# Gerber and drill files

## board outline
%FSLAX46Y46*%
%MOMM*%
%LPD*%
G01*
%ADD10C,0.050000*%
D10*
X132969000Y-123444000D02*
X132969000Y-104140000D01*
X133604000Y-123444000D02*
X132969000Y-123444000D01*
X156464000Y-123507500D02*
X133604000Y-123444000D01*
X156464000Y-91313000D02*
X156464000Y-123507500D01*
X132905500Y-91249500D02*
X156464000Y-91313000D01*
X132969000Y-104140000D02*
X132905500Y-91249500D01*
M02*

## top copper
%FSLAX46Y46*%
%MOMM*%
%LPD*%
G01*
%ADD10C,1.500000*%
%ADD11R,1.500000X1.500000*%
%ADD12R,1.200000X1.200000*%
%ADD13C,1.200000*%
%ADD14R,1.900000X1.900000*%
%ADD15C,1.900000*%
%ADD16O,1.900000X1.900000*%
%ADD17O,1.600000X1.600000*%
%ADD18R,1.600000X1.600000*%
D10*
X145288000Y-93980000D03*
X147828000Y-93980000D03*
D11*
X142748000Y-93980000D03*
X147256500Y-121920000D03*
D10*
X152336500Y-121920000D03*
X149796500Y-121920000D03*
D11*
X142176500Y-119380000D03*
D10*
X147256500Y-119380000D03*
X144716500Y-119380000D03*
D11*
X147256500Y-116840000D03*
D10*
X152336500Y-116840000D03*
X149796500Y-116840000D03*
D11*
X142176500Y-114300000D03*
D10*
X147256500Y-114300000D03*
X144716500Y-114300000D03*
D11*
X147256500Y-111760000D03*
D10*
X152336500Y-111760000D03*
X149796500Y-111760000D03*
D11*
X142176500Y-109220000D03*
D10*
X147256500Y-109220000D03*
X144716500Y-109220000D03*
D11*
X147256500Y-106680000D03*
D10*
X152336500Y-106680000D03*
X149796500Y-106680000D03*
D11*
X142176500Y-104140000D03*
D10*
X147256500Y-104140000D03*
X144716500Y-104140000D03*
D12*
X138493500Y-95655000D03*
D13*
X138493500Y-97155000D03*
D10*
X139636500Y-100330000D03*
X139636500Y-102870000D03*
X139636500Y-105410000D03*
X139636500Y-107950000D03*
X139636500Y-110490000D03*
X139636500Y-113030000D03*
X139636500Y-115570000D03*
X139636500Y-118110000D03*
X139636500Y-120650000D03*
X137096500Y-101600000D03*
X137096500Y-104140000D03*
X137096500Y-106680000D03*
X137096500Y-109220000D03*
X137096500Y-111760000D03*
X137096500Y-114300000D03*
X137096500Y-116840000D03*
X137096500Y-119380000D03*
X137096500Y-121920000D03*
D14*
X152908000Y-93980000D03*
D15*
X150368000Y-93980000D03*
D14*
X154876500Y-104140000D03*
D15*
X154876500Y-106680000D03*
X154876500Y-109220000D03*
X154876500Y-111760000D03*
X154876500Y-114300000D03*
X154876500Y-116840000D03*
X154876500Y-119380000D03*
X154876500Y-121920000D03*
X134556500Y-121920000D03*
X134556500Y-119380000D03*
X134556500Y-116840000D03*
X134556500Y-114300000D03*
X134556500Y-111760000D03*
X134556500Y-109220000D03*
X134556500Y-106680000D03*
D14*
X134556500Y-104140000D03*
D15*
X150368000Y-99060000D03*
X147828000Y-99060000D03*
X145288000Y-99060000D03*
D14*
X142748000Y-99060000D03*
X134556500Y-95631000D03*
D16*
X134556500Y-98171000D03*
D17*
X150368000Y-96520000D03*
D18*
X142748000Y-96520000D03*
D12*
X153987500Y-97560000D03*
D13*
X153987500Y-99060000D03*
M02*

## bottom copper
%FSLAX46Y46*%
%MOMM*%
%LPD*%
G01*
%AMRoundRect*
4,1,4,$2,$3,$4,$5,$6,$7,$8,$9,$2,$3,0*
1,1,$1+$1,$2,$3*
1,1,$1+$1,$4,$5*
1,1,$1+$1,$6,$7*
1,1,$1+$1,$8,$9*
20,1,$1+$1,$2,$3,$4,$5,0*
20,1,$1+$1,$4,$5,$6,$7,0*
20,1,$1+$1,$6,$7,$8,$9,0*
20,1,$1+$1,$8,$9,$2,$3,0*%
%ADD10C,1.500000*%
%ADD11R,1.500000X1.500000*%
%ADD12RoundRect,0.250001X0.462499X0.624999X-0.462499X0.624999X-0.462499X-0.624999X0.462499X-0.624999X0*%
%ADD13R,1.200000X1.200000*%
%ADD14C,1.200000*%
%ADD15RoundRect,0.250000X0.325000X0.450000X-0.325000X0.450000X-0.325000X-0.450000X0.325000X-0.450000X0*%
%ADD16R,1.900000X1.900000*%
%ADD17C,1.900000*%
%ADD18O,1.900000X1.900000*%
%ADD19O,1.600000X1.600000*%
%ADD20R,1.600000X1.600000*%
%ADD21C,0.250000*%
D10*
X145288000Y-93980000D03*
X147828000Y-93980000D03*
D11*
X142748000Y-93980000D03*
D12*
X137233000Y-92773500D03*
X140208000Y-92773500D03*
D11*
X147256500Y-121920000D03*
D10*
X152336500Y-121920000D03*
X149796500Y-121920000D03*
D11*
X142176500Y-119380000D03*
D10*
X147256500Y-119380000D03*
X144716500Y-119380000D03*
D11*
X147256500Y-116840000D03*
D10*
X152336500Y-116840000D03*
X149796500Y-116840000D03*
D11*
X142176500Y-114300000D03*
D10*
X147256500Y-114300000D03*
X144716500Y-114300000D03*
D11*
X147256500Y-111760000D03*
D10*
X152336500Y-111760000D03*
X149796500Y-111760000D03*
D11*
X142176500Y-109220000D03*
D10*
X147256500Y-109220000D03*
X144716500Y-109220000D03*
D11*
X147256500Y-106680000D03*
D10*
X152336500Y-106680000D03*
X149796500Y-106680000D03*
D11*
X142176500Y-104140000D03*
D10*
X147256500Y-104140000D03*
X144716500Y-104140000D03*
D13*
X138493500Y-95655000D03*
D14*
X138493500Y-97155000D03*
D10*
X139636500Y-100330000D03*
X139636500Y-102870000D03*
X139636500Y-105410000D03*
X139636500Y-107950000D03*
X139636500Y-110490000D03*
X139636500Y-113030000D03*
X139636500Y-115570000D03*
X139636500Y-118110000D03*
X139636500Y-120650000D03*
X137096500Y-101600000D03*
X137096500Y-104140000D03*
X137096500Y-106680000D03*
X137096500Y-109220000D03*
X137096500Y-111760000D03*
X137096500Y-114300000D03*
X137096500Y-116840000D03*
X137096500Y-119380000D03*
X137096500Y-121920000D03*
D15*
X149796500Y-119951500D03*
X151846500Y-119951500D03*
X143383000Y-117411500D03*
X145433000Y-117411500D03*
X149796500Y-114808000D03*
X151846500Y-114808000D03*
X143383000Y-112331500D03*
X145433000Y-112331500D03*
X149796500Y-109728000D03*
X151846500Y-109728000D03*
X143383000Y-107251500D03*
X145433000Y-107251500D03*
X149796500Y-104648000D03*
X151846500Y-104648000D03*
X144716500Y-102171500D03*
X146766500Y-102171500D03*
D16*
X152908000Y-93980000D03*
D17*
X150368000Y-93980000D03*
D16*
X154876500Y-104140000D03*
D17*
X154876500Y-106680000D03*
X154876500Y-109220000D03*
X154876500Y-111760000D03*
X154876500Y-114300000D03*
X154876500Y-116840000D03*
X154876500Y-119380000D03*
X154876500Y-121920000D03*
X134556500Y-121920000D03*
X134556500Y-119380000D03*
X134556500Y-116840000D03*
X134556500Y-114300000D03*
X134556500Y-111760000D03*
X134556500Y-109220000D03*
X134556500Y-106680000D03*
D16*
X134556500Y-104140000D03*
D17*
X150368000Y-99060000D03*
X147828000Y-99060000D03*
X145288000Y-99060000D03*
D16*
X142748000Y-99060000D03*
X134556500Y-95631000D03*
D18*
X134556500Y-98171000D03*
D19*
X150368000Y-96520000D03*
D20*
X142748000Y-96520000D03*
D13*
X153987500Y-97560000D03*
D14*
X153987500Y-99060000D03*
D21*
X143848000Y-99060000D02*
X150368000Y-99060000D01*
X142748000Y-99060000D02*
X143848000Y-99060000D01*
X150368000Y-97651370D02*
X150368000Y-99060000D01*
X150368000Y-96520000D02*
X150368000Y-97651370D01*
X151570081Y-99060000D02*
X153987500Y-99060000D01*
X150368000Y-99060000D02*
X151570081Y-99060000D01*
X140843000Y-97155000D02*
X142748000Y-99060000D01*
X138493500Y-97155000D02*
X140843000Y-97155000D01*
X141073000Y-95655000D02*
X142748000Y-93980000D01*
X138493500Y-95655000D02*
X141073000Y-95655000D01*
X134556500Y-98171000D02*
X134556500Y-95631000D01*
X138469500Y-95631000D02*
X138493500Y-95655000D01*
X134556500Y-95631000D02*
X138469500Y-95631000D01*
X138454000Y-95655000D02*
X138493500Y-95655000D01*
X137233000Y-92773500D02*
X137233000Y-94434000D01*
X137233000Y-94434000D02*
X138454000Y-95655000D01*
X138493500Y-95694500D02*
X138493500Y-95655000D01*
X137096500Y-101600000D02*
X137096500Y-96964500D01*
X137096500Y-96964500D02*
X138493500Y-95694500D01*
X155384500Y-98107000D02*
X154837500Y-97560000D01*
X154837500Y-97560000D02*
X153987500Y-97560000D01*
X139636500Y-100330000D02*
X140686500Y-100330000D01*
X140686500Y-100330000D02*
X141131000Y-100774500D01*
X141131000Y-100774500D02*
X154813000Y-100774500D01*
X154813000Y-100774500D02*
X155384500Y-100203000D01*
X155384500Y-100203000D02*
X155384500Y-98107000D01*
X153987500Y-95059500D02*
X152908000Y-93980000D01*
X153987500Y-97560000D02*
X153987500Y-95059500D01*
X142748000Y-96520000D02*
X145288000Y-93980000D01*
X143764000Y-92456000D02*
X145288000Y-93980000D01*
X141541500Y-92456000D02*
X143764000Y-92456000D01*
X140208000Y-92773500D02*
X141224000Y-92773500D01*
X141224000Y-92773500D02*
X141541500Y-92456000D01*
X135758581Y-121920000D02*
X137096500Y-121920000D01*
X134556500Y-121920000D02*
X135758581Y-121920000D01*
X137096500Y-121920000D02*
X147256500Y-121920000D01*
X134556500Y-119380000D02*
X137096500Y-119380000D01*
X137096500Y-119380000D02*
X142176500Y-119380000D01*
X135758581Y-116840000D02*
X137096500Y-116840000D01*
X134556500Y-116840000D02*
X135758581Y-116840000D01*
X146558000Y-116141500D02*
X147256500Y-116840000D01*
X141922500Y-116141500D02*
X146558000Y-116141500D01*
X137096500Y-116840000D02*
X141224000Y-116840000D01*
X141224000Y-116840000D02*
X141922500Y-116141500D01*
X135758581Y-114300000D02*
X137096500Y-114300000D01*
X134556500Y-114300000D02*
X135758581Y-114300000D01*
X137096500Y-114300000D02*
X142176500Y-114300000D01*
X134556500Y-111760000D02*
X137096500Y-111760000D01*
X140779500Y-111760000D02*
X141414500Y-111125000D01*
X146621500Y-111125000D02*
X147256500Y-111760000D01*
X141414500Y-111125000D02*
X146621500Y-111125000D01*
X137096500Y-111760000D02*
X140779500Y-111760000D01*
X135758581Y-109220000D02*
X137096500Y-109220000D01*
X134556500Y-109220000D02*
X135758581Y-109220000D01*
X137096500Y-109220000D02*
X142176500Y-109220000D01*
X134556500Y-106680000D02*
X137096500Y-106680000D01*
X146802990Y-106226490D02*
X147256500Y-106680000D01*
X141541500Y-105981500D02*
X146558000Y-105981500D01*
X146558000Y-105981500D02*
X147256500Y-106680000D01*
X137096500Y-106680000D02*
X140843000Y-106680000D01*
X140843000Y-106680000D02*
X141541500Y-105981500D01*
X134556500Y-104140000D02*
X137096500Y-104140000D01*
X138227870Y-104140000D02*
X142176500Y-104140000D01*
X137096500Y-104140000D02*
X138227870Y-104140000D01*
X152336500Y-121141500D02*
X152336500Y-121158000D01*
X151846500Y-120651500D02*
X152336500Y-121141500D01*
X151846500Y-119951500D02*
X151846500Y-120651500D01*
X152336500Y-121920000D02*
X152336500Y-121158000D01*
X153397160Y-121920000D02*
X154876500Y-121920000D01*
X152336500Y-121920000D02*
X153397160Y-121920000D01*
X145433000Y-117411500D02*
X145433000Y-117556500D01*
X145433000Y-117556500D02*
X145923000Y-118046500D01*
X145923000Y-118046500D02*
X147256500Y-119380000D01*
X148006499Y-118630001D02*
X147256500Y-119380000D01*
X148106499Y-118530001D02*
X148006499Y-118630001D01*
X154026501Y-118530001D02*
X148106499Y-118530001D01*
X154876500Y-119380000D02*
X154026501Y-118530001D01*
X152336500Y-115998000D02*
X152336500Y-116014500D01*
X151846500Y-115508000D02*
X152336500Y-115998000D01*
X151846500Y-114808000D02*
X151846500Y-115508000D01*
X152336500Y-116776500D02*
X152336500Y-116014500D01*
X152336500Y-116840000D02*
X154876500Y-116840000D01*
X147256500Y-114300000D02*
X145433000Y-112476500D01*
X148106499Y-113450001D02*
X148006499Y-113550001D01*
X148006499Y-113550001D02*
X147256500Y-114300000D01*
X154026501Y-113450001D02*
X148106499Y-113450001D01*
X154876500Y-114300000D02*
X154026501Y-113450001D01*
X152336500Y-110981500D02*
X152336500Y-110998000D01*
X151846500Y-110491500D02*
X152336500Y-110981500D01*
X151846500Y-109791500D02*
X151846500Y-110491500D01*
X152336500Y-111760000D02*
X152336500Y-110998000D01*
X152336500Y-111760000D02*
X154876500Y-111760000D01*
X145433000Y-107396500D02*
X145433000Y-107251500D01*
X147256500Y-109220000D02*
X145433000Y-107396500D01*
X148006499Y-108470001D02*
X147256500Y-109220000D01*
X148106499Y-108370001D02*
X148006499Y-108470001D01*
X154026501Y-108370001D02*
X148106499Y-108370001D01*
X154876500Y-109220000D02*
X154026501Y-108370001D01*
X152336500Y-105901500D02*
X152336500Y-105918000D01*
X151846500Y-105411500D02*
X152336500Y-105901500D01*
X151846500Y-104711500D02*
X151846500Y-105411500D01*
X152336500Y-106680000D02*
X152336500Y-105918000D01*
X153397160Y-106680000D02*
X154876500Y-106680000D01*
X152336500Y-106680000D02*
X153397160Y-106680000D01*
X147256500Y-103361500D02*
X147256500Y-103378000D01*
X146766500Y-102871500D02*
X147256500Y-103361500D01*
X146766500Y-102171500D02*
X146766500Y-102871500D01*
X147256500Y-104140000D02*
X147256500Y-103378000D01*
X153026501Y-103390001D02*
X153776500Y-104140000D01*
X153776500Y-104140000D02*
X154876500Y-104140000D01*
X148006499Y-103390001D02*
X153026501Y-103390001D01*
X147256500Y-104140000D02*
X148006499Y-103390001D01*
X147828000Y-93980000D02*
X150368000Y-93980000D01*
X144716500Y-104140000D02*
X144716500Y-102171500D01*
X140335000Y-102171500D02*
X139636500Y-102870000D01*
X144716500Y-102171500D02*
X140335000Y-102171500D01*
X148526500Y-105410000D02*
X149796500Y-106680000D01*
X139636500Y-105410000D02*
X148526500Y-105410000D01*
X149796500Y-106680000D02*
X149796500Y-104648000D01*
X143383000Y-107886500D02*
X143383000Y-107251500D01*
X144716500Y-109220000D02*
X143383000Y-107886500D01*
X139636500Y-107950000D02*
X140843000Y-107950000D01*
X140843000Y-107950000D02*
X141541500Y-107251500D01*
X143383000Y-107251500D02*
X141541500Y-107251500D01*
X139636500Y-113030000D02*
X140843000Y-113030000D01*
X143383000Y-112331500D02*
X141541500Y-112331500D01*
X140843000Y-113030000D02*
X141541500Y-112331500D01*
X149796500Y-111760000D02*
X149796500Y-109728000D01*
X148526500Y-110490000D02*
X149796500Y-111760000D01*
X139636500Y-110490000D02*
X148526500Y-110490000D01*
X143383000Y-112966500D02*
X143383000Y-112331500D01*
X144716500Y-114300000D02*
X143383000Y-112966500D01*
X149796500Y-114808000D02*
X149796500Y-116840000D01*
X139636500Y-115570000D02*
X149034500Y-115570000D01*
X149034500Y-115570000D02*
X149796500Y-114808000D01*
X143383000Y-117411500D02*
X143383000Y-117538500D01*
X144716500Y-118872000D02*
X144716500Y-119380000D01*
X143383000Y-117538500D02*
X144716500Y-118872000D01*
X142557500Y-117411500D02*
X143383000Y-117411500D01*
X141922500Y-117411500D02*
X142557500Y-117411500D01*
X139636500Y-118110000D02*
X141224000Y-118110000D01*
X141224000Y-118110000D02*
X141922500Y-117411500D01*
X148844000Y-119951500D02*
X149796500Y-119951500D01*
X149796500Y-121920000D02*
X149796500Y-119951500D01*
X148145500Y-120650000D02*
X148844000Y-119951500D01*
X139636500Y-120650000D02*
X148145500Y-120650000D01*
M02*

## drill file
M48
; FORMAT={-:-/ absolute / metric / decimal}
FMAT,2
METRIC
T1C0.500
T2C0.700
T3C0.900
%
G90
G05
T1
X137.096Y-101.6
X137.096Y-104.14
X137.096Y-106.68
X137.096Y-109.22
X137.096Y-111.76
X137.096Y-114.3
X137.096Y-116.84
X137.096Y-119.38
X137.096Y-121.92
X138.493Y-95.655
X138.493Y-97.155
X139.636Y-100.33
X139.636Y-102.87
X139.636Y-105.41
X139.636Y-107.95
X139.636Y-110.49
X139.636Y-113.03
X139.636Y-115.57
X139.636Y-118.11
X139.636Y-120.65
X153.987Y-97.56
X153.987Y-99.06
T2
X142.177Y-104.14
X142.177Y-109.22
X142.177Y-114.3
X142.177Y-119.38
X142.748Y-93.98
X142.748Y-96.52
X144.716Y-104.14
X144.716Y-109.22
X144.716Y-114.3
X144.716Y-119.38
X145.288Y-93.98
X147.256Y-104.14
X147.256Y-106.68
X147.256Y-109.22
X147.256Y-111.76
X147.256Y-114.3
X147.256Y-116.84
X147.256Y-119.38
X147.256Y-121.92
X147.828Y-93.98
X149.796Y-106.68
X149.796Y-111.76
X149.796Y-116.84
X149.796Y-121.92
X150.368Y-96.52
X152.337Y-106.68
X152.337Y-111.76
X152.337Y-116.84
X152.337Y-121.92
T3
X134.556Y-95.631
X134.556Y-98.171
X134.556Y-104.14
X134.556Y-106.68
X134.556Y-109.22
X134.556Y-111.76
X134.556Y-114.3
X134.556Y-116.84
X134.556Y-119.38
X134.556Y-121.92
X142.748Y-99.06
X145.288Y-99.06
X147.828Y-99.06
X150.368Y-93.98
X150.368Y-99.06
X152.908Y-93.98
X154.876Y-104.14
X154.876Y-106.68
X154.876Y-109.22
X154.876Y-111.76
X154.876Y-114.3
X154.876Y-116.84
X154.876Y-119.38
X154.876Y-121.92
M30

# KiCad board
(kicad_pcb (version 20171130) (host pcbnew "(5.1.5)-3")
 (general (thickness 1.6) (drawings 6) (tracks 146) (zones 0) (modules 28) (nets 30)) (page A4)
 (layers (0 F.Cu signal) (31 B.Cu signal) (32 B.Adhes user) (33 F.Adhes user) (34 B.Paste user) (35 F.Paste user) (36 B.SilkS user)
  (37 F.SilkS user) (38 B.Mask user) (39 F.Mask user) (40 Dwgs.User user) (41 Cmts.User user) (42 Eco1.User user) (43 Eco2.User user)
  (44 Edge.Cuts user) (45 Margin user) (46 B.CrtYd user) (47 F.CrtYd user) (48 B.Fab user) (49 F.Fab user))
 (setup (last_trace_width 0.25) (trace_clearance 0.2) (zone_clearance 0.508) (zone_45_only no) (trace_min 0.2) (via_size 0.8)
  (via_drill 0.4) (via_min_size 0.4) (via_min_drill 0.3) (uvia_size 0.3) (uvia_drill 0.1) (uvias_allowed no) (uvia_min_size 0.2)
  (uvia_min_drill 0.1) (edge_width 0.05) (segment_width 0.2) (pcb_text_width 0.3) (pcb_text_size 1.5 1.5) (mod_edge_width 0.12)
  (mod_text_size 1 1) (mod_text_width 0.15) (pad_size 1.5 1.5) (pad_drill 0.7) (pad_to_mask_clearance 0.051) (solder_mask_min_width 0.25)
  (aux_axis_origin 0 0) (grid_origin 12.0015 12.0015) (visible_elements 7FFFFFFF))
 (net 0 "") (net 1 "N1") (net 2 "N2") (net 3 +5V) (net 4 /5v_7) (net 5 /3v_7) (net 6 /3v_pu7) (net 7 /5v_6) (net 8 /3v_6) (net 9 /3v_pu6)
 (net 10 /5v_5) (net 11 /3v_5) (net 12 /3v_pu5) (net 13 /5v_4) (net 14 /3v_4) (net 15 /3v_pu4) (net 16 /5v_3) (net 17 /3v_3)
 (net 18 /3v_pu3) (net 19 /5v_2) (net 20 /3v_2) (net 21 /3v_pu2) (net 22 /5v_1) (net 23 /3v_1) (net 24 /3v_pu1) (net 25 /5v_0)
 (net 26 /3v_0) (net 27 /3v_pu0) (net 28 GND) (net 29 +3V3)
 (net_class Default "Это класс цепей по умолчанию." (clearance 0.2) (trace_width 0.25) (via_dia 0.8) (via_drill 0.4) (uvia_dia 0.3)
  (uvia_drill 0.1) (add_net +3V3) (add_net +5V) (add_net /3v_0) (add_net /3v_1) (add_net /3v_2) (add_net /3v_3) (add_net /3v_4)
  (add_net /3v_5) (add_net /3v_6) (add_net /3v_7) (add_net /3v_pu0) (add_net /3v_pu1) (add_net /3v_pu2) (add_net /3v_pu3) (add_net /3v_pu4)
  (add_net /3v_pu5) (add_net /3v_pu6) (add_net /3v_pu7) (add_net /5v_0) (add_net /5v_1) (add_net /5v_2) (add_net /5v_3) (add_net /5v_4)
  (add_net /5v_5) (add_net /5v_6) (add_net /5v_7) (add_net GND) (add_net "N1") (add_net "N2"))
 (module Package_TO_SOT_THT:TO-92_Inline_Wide (layer F.Cu) (at 142.748 93.98)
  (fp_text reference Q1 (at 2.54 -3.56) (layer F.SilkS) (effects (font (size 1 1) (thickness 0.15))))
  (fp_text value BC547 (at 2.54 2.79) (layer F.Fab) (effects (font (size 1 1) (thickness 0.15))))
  (pad 2 thru_hole circle (at 2.54 0 90) (size 1.5 1.5) (drill 0.7) (layers *.Cu *.Mask) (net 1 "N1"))
  (pad 3 thru_hole circle (at 5.08 0 90) (size 1.5 1.5) (drill 0.7) (layers *.Cu *.Mask) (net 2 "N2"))
  (pad 1 thru_hole rect (at 0 0 90) (size 1.5 1.5) (drill 0.7) (layers *.Cu *.Mask) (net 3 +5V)))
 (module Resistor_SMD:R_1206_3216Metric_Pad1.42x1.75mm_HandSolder (layer B.Cu) (at 138.7205 92.7735 180)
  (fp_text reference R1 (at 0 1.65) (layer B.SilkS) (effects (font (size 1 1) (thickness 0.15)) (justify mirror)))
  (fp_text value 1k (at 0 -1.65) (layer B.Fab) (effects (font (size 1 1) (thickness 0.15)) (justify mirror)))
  (pad 2 smd roundrect (at 1.4875 0 180) (size 1.425 1.75) (layers B.Cu B.Paste B.Mask) (roundrect_rratio 0.175439) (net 3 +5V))
  (pad 1 smd roundrect (at -1.4875 0 180) (size 1.425 1.75) (layers B.Cu B.Paste B.Mask) (roundrect_rratio 0.175439) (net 1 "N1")))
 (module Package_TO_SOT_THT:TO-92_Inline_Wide (layer F.Cu) (at 147.2565 121.92)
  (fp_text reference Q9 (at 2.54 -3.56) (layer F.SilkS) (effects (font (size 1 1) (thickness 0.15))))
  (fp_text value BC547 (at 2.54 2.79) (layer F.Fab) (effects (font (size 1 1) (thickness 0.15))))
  (pad 1 thru_hole rect (at 0 0 90) (size 1.5 1.5) (drill 0.7) (layers *.Cu *.Mask) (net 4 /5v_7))
  (pad 3 thru_hole circle (at 5.08 0 90) (size 1.5 1.5) (drill 0.7) (layers *.Cu *.Mask) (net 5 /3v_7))
  (pad 2 thru_hole circle (at 2.54 0 90) (size 1.5 1.5) (drill 0.7) (layers *.Cu *.Mask) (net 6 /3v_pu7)))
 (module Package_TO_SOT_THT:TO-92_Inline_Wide (layer F.Cu) (at 142.1765 119.38)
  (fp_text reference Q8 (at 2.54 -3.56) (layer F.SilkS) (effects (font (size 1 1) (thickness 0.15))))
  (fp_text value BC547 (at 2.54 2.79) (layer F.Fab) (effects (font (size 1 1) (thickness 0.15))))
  (pad 1 thru_hole rect (at 0 0 90) (size 1.5 1.5) (drill 0.7) (layers *.Cu *.Mask) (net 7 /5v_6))
  (pad 3 thru_hole circle (at 5.08 0 90) (size 1.5 1.5) (drill 0.7) (layers *.Cu *.Mask) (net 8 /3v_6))
  (pad 2 thru_hole circle (at 2.54 0 90) (size 1.5 1.5) (drill 0.7) (layers *.Cu *.Mask) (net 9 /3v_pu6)))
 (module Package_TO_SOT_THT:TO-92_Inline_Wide (layer F.Cu) (at 147.2565 116.84)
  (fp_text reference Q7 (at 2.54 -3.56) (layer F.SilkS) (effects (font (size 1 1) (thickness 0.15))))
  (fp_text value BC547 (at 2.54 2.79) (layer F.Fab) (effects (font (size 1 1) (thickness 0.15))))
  (pad 1 thru_hole rect (at 0 0 90) (size 1.5 1.5) (drill 0.7) (layers *.Cu *.Mask) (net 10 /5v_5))
  (pad 3 thru_hole circle (at 5.08 0 90) (size 1.5 1.5) (drill 0.7) (layers *.Cu *.Mask) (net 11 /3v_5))
  (pad 2 thru_hole circle (at 2.54 0 90) (size 1.5 1.5) (drill 0.7) (layers *.Cu *.Mask) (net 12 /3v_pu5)))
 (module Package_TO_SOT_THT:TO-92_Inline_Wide (layer F.Cu) (at 142.1765 114.3)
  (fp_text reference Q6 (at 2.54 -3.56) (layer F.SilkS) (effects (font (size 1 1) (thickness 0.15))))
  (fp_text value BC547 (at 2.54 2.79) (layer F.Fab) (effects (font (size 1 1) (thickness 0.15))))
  (pad 1 thru_hole rect (at 0 0 90) (size 1.5 1.5) (drill 0.7) (layers *.Cu *.Mask) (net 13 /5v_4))
  (pad 3 thru_hole circle (at 5.08 0 90) (size 1.5 1.5) (drill 0.7) (layers *.Cu *.Mask) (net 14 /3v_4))
  (pad 2 thru_hole circle (at 2.54 0 90) (size 1.5 1.5) (drill 0.7) (layers *.Cu *.Mask) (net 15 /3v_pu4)))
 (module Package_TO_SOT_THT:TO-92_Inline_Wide (layer F.Cu) (at 147.2565 111.76)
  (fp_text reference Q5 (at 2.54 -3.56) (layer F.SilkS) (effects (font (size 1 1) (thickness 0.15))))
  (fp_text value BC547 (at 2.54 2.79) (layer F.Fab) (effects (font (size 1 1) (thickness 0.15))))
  (pad 1 thru_hole rect (at 0 0 90) (size 1.5 1.5) (drill 0.7) (layers *.Cu *.Mask) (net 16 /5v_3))
  (pad 3 thru_hole circle (at 5.08 0 90) (size 1.5 1.5) (drill 0.7) (layers *.Cu *.Mask) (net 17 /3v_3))
  (pad 2 thru_hole circle (at 2.54 0 90) (size 1.5 1.5) (drill 0.7) (layers *.Cu *.Mask) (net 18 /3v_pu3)))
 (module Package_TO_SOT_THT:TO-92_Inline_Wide (layer F.Cu) (at 142.1765 109.22)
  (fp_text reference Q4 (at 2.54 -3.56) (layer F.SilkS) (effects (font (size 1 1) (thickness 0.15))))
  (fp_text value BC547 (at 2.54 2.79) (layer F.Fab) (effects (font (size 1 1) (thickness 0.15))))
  (pad 1 thru_hole rect (at 0 0 90) (size 1.5 1.5) (drill 0.7) (layers *.Cu *.Mask) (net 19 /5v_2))
  (pad 3 thru_hole circle (at 5.08 0 90) (size 1.5 1.5) (drill 0.7) (layers *.Cu *.Mask) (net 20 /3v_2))
  (pad 2 thru_hole circle (at 2.54 0 90) (size 1.5 1.5) (drill 0.7) (layers *.Cu *.Mask) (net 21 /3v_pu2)))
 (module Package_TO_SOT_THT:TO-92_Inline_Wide (layer F.Cu) (at 147.2565 106.68)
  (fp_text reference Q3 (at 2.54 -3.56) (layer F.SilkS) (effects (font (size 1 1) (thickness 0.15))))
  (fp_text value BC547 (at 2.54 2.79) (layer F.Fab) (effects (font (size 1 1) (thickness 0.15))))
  (pad 1 thru_hole rect (at 0 0 90) (size 1.5 1.5) (drill 0.7) (layers *.Cu *.Mask) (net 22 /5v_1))
  (pad 3 thru_hole circle (at 5.08 0 90) (size 1.5 1.5) (drill 0.7) (layers *.Cu *.Mask) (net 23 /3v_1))
  (pad 2 thru_hole circle (at 2.54 0 90) (size 1.5 1.5) (drill 0.7) (layers *.Cu *.Mask) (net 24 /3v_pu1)))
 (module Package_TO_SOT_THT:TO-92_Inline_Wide (layer F.Cu) (at 142.1765 104.14)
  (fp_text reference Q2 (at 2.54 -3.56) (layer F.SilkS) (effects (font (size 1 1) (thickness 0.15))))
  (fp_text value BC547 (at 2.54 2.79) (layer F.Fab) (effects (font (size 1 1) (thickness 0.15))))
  (pad 1 thru_hole rect (at 0 0 90) (size 1.5 1.5) (drill 0.7) (layers *.Cu *.Mask) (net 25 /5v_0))
  (pad 3 thru_hole circle (at 5.08 0 90) (size 1.5 1.5) (drill 0.7) (layers *.Cu *.Mask) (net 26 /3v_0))
  (pad 2 thru_hole circle (at 2.54 0 90) (size 1.5 1.5) (drill 0.7) (layers *.Cu *.Mask) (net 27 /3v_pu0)))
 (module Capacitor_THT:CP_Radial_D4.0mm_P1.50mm (layer F.Cu) (at 138.4935 95.655 270)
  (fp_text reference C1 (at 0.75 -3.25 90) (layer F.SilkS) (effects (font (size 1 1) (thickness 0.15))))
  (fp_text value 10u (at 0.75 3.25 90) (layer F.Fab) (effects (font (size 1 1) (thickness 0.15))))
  (pad 1 thru_hole rect (at 0 0 270) (size 1.2 1.2) (drill 0.5) (layers *.Cu *.Mask) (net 3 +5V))
  (pad 2 thru_hole circle (at 1.5 0 270) (size 1.2 1.2) (drill 0.5) (layers *.Cu *.Mask) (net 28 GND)))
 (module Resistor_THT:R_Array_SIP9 (layer F.Cu) (at 139.6365 100.33 270)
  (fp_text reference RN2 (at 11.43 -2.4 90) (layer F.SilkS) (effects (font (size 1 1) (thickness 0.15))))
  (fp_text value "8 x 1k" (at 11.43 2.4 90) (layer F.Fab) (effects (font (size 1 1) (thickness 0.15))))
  (pad 1 thru_hole circle (at 0 0 270) (size 1.5 1.5) (drill 0.5) (layers *.Cu *.Mask) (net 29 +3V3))
  (pad 2 thru_hole circle (at 2.54 0 270) (size 1.5 1.5) (drill 0.5) (layers *.Cu *.Mask) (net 27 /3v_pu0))
  (pad 3 thru_hole circle (at 5.08 0 270) (size 1.5 1.5) (drill 0.5) (layers *.Cu *.Mask) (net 24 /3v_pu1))
  (pad 4 thru_hole circle (at 7.62 0 270) (size 1.5 1.5) (drill 0.5) (layers *.Cu *.Mask) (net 21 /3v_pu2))
  (pad 5 thru_hole circle (at 10.16 0 270) (size 1.5 1.5) (drill 0.5) (layers *.Cu *.Mask) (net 18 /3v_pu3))
  (pad 6 thru_hole circle (at 12.7 0 270) (size 1.5 1.5) (drill 0.5) (layers *.Cu *.Mask) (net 15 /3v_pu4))
  (pad 7 thru_hole circle (at 15.24 0 270) (size 1.5 1.5) (drill 0.5) (layers *.Cu *.Mask) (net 12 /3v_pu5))
  (pad 8 thru_hole circle (at 17.78 0 270) (size 1.5 1.5) (drill 0.5) (layers *.Cu *.Mask) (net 9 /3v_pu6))
  (pad 9 thru_hole circle (at 20.32 0 270) (size 1.5 1.5) (drill 0.5) (layers *.Cu *.Mask) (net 6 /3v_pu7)))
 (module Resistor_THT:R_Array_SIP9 (layer F.Cu) (at 137.0965 101.6 270)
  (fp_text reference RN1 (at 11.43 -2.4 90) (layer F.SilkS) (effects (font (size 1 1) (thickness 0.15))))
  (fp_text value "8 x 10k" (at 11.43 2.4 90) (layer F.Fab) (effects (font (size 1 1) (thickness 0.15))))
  (pad 1 thru_hole circle (at 0 0 270) (size 1.5 1.5) (drill 0.5) (layers *.Cu *.Mask) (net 3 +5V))
  (pad 2 thru_hole circle (at 2.54 0 270) (size 1.5 1.5) (drill 0.5) (layers *.Cu *.Mask) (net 25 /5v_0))
  (pad 3 thru_hole circle (at 5.08 0 270) (size 1.5 1.5) (drill 0.5) (layers *.Cu *.Mask) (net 22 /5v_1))
  (pad 4 thru_hole circle (at 7.62 0 270) (size 1.5 1.5) (drill 0.5) (layers *.Cu *.Mask) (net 19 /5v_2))
  (pad 5 thru_hole circle (at 10.16 0 270) (size 1.5 1.5) (drill 0.5) (layers *.Cu *.Mask) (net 16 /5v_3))
  (pad 6 thru_hole circle (at 12.7 0 270) (size 1.5 1.5) (drill 0.5) (layers *.Cu *.Mask) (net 13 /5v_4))
  (pad 7 thru_hole circle (at 15.24 0 270) (size 1.5 1.5) (drill 0.5) (layers *.Cu *.Mask) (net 10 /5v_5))
  (pad 8 thru_hole circle (at 17.78 0 270) (size 1.5 1.5) (drill 0.5) (layers *.Cu *.Mask) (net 7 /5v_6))
  (pad 9 thru_hole circle (at 20.32 0 270) (size 1.5 1.5) (drill 0.5) (layers *.Cu *.Mask) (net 4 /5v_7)))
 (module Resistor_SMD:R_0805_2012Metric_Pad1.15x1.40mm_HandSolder (layer B.Cu) (at 150.8215 119.9515 180)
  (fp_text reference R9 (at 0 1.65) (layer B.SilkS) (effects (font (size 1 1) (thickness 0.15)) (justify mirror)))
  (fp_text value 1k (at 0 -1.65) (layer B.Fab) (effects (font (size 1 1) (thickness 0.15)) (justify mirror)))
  (pad 2 smd roundrect (at 1.025 0 180) (size 1.15 1.4) (layers B.Cu B.Paste B.Mask) (roundrect_rratio 0.217391) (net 6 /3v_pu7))
  (pad 1 smd roundrect (at -1.025 0 180) (size 1.15 1.4) (layers B.Cu B.Paste B.Mask) (roundrect_rratio 0.217391) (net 5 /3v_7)))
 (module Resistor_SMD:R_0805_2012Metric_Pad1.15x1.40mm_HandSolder (layer B.Cu) (at 144.408 117.4115 180)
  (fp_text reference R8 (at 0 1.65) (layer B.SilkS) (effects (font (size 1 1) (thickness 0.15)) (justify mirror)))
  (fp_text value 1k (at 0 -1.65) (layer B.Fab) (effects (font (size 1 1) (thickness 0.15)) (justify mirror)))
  (pad 2 smd roundrect (at 1.025 0 180) (size 1.15 1.4) (layers B.Cu B.Paste B.Mask) (roundrect_rratio 0.217391) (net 9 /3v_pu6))
  (pad 1 smd roundrect (at -1.025 0 180) (size 1.15 1.4) (layers B.Cu B.Paste B.Mask) (roundrect_rratio 0.217391) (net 8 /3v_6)))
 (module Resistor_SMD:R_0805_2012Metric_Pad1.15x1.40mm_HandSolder (layer B.Cu) (at 150.8215 114.808 180)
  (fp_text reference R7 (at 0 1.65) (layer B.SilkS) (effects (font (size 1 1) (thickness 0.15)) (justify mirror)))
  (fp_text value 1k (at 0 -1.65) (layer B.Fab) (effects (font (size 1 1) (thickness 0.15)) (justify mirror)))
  (pad 2 smd roundrect (at 1.025 0 180) (size 1.15 1.4) (layers B.Cu B.Paste B.Mask) (roundrect_rratio 0.217391) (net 12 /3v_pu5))
  (pad 1 smd roundrect (at -1.025 0 180) (size 1.15 1.4) (layers B.Cu B.Paste B.Mask) (roundrect_rratio 0.217391) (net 11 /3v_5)))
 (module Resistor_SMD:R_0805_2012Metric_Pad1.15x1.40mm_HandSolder (layer B.Cu) (at 144.408 112.3315 180)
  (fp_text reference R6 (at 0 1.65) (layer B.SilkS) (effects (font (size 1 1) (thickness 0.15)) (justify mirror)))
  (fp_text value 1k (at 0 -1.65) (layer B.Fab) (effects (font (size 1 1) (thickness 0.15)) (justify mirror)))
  (pad 2 smd roundrect (at 1.025 0 180) (size 1.15 1.4) (layers B.Cu B.Paste B.Mask) (roundrect_rratio 0.217391) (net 15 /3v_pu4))
  (pad 1 smd roundrect (at -1.025 0 180) (size 1.15 1.4) (layers B.Cu B.Paste B.Mask) (roundrect_rratio 0.217391) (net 14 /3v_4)))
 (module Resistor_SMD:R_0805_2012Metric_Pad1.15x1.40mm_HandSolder (layer B.Cu) (at 150.8215 109.728 180)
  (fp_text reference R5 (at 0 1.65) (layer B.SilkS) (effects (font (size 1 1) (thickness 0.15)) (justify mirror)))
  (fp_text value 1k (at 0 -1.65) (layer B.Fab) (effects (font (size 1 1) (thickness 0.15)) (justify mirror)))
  (pad 2 smd roundrect (at 1.025 0 180) (size 1.15 1.4) (layers B.Cu B.Paste B.Mask) (roundrect_rratio 0.217391) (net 18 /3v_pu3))
  (pad 1 smd roundrect (at -1.025 0 180) (size 1.15 1.4) (layers B.Cu B.Paste B.Mask) (roundrect_rratio 0.217391) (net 17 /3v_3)))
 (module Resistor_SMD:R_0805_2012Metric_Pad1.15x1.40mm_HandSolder (layer B.Cu) (at 144.408 107.2515 180)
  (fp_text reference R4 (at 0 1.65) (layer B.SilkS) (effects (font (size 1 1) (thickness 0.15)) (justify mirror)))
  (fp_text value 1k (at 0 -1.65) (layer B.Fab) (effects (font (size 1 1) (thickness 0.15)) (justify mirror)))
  (pad 2 smd roundrect (at 1.025 0 180) (size 1.15 1.4) (layers B.Cu B.Paste B.Mask) (roundrect_rratio 0.217391) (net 21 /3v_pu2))
  (pad 1 smd roundrect (at -1.025 0 180) (size 1.15 1.4) (layers B.Cu B.Paste B.Mask) (roundrect_rratio 0.217391) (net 20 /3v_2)))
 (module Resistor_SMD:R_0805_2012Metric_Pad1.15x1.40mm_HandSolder (layer B.Cu) (at 150.8215 104.648 180)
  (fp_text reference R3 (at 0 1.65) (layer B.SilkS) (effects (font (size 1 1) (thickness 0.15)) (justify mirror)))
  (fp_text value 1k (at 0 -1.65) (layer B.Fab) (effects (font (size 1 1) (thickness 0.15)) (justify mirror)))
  (pad 2 smd roundrect (at 1.025 0 180) (size 1.15 1.4) (layers B.Cu B.Paste B.Mask) (roundrect_rratio 0.217391) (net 24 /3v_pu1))
  (pad 1 smd roundrect (at -1.025 0 180) (size 1.15 1.4) (layers B.Cu B.Paste B.Mask) (roundrect_rratio 0.217391) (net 23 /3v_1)))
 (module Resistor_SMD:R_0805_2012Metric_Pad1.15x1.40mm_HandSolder (layer B.Cu) (at 145.7415 102.1715 180)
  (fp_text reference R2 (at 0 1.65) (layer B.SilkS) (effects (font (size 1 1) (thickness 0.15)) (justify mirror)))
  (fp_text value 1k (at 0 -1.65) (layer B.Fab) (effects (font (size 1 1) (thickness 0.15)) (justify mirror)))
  (pad 2 smd roundrect (at 1.025 0 180) (size 1.15 1.4) (layers B.Cu B.Paste B.Mask) (roundrect_rratio 0.217391) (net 27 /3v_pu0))
  (pad 1 smd roundrect (at -1.025 0 180) (size 1.15 1.4) (layers B.Cu B.Paste B.Mask) (roundrect_rratio 0.217391) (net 26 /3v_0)))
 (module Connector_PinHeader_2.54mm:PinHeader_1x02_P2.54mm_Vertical (layer F.Cu) (at 152.908 93.98 270)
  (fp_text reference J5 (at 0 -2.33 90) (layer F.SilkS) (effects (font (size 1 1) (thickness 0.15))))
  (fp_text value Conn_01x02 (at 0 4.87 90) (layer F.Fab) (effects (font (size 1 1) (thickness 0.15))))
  (pad 1 thru_hole rect (at 0 0 270) (size 1.9 1.9) (drill 0.9) (layers *.Cu *.Mask) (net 29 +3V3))
  (pad 2 thru_hole circle (at 0 2.54 270) (size 1.9 1.9) (drill 0.9) (layers *.Cu *.Mask) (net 2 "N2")))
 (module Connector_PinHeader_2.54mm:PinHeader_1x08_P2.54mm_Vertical (layer F.Cu) (at 154.8765 104.14)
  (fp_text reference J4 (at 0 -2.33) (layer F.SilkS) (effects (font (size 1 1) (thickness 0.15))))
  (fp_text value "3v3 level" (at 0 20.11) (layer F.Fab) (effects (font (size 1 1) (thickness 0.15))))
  (pad 1 thru_hole rect (at 0 0) (size 1.9 1.9) (drill 0.9) (layers *.Cu *.Mask) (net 26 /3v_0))
  (pad 2 thru_hole circle (at 0 2.54) (size 1.9 1.9) (drill 0.9) (layers *.Cu *.Mask) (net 23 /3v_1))
  (pad 3 thru_hole circle (at 0 5.08) (size 1.9 1.9) (drill 0.9) (layers *.Cu *.Mask) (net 20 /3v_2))
  (pad 4 thru_hole circle (at 0 7.62) (size 1.9 1.9) (drill 0.9) (layers *.Cu *.Mask) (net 17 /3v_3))
  (pad 5 thru_hole circle (at 0 10.16) (size 1.9 1.9) (drill 0.9) (layers *.Cu *.Mask) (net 14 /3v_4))
  (pad 6 thru_hole circle (at 0 12.7) (size 1.9 1.9) (drill 0.9) (layers *.Cu *.Mask) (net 11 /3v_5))
  (pad 7 thru_hole circle (at 0 15.24) (size 1.9 1.9) (drill 0.9) (layers *.Cu *.Mask) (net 8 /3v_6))
  (pad 8 thru_hole circle (at 0 17.78) (size 1.9 1.9) (drill 0.9) (layers *.Cu *.Mask) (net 5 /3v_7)))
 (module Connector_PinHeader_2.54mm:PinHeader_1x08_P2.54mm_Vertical (layer F.Cu) (at 134.5565 104.14)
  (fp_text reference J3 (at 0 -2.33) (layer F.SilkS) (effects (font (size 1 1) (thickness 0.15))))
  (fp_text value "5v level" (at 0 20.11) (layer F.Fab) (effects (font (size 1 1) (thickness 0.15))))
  (pad 8 thru_hole circle (at 0 17.78) (size 1.9 1.9) (drill 0.9) (layers *.Cu *.Mask) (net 4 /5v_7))
  (pad 7 thru_hole circle (at 0 15.24) (size 1.9 1.9) (drill 0.9) (layers *.Cu *.Mask) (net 7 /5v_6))
  (pad 6 thru_hole circle (at 0 12.7) (size 1.9 1.9) (drill 0.9) (layers *.Cu *.Mask) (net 10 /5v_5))
  (pad 5 thru_hole circle (at 0 10.16) (size 1.9 1.9) (drill 0.9) (layers *.Cu *.Mask) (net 13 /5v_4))
  (pad 4 thru_hole circle (at 0 7.62) (size 1.9 1.9) (drill 0.9) (layers *.Cu *.Mask) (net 16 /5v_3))
  (pad 3 thru_hole circle (at 0 5.08) (size 1.9 1.9) (drill 0.9) (layers *.Cu *.Mask) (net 19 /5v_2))
  (pad 2 thru_hole circle (at 0 2.54) (size 1.9 1.9) (drill 0.9) (layers *.Cu *.Mask) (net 22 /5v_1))
  (pad 1 thru_hole rect (at 0 0) (size 1.9 1.9) (drill 0.9) (layers *.Cu *.Mask) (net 25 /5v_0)))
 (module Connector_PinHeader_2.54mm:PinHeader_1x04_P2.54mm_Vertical (layer F.Cu) (at 142.748 99.06 90)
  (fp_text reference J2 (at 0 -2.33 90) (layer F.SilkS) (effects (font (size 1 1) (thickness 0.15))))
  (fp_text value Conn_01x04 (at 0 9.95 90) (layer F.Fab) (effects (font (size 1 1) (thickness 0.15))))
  (pad 4 thru_hole circle (at 0 7.62 90) (size 1.9 1.9) (drill 0.9) (layers *.Cu *.Mask) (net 28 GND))
  (pad 3 thru_hole circle (at 0 5.08 90) (size 1.9 1.9) (drill 0.9) (layers *.Cu *.Mask) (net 28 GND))
  (pad 2 thru_hole circle (at 0 2.54 90) (size 1.9 1.9) (drill 0.9) (layers *.Cu *.Mask) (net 28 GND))
  (pad 1 thru_hole rect (at 0 0 90) (size 1.9 1.9) (drill 0.9) (layers *.Cu *.Mask) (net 28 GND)))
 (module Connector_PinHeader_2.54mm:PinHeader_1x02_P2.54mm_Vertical (layer F.Cu) (at 134.5565 95.631)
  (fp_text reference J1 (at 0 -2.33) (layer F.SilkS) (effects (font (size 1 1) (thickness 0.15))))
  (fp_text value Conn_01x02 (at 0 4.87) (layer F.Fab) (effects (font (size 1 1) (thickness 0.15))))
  (pad 1 thru_hole rect (at 0 0) (size 1.9 1.9) (drill 0.9) (layers *.Cu *.Mask) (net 3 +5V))
  (pad 2 thru_hole oval (at 0 2.54) (size 1.9 1.9) (drill 0.9) (layers *.Cu *.Mask) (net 3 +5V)))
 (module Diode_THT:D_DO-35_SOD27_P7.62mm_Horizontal (layer F.Cu) (at 142.748 96.52)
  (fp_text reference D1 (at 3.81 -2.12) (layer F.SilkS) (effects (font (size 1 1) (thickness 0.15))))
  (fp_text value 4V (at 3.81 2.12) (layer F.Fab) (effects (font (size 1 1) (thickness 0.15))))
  (pad 2 thru_hole oval (at 7.62 0) (size 1.6 1.6) (drill 0.7) (layers *.Cu *.Mask) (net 28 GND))
  (pad 1 thru_hole rect (at 0 0) (size 1.6 1.6) (drill 0.7) (layers *.Cu *.Mask) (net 1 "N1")))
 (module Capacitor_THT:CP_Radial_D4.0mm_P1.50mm (layer F.Cu) (at 153.9875 97.56 270)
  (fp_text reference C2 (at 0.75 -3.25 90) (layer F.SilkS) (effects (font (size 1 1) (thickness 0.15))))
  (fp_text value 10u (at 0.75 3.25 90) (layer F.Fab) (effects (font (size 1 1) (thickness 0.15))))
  (pad 1 thru_hole rect (at 0 0 270) (size 1.2 1.2) (drill 0.5) (layers *.Cu *.Mask) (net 29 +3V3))
  (pad 2 thru_hole circle (at 1.5 0 270) (size 1.2 1.2) (drill 0.5) (layers *.Cu *.Mask) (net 28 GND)))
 (gr_line (start 132.969 123.444) (end 132.969 104.14) (layer Edge.Cuts) (width 0.05))
 (gr_line (start 133.604 123.444) (end 132.969 123.444) (layer Edge.Cuts) (width 0.05))
 (gr_line (start 156.464 123.5075) (end 133.604 123.444) (layer Edge.Cuts) (width 0.05))
 (gr_line (start 156.464 91.313) (end 156.464 123.5075) (layer Edge.Cuts) (width 0.05))
 (gr_line (start 132.9055 91.2495) (end 156.464 91.313) (layer Edge.Cuts) (width 0.05))
 (gr_line (start 132.969 104.14) (end 132.9055 91.2495) (layer Edge.Cuts) (width 0.05))
 (segment (start 143.848 99.06) (end 150.368 99.06) (width 0.25) (layer B.Cu) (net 28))
 (segment (start 142.748 99.06) (end 143.848 99.06) (width 0.25) (layer B.Cu) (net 28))
 (segment (start 150.368 97.65137) (end 150.368 99.06) (width 0.25) (layer B.Cu) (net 28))
 (segment (start 150.368 96.52) (end 150.368 97.65137) (width 0.25) (layer B.Cu) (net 28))
 (segment (start 151.570081 99.06) (end 153.9875 99.06) (width 0.25) (layer B.Cu) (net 28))
 (segment (start 150.368 99.06) (end 151.570081 99.06) (width 0.25) (layer B.Cu) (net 28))
 (segment (start 140.843 97.155) (end 142.748 99.06) (width 0.25) (layer B.Cu) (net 28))
 (segment (start 138.4935 97.155) (end 140.843 97.155) (width 0.25) (layer B.Cu) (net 28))
 (segment (start 141.073 95.655) (end 142.748 93.98) (width 0.25) (layer B.Cu) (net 3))
 (segment (start 138.4935 95.655) (end 141.073 95.655) (width 0.25) (layer B.Cu) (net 3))
 (segment (start 134.5565 98.171) (end 134.5565 95.631) (width 0.25) (layer B.Cu) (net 3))
 (segment (start 138.4695 95.631) (end 138.4935 95.655) (width 0.25) (layer B.Cu) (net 3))
 (segment (start 134.5565 95.631) (end 138.4695 95.631) (width 0.25) (layer B.Cu) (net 3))
 (segment (start 138.454 95.655) (end 138.4935 95.655) (width 0.25) (layer B.Cu) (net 3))
 (segment (start 137.233 92.7735) (end 137.233 94.434) (width 0.25) (layer B.Cu) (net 3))
 (segment (start 137.233 94.434) (end 138.454 95.655) (width 0.25) (layer B.Cu) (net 3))
 (segment (start 138.4935 95.6945) (end 138.4935 95.655) (width 0.25) (layer B.Cu) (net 3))
 (segment (start 137.0965 101.6) (end 137.0965 96.9645) (width 0.25) (layer B.Cu) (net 3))
 (segment (start 137.0965 96.9645) (end 138.4935 95.6945) (width 0.25) (layer B.Cu) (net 3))
 (segment (start 155.3845 98.107) (end 154.8375 97.56) (width 0.25) (layer B.Cu) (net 29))
 (segment (start 154.8375 97.56) (end 153.9875 97.56) (width 0.25) (layer B.Cu) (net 29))
 (segment (start 139.6365 100.33) (end 140.6865 100.33) (width 0.25) (layer B.Cu) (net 29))
 (segment (start 140.6865 100.33) (end 141.131 100.7745) (width 0.25) (layer B.Cu) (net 29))
 (segment (start 141.131 100.7745) (end 154.813 100.7745) (width 0.25) (layer B.Cu) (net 29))
 (segment (start 154.813 100.7745) (end 155.3845 100.203) (width 0.25) (layer B.Cu) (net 29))
 (segment (start 155.3845 100.203) (end 155.3845 98.107) (width 0.25) (layer B.Cu) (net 29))
 (segment (start 153.9875 95.0595) (end 152.908 93.98) (width 0.25) (layer B.Cu) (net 29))
 (segment (start 153.9875 97.56) (end 153.9875 95.0595) (width 0.25) (layer B.Cu) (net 29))
 (segment (start 142.748 96.52) (end 145.288 93.98) (width 0.25) (layer B.Cu) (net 1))
 (segment (start 143.764 92.456) (end 145.288 93.98) (width 0.25) (layer B.Cu) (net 1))
 (segment (start 141.5415 92.456) (end 143.764 92.456) (width 0.25) (layer B.Cu) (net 1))
 (segment (start 140.208 92.7735) (end 141.224 92.7735) (width 0.25) (layer B.Cu) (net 1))
 (segment (start 141.224 92.7735) (end 141.5415 92.456) (width 0.25) (layer B.Cu) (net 1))
 (segment (start 135.758581 121.92) (end 137.0965 121.92) (width 0.25) (layer B.Cu) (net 4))
 (segment (start 134.5565 121.92) (end 135.758581 121.92) (width 0.25) (layer B.Cu) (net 4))
 (segment (start 137.0965 121.92) (end 147.2565 121.92) (width 0.25) (layer B.Cu) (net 4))
 (segment (start 134.5565 119.38) (end 137.0965 119.38) (width 0.25) (layer B.Cu) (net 7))
 (segment (start 137.0965 119.38) (end 142.1765 119.38) (width 0.25) (layer B.Cu) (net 7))
 (segment (start 135.758581 116.84) (end 137.0965 116.84) (width 0.25) (layer B.Cu) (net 10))
 (segment (start 134.5565 116.84) (end 135.758581 116.84) (width 0.25) (layer B.Cu) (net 10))
 (segment (start 146.558 116.1415) (end 147.2565 116.84) (width 0.25) (layer B.Cu) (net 10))
 (segment (start 141.9225 116.1415) (end 146.558 116.1415) (width 0.25) (layer B.Cu) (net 10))
 (segment (start 137.0965 116.84) (end 141.224 116.84) (width 0.25) (layer B.Cu) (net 10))
 (segment (start 141.224 116.84) (end 141.9225 116.1415) (width 0.25) (layer B.Cu) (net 10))
 (segment (start 135.758581 114.3) (end 137.0965 114.3) (width 0.25) (layer B.Cu) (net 13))
 (segment (start 134.5565 114.3) (end 135.758581 114.3) (width 0.25) (layer B.Cu) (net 13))
 (segment (start 137.0965 114.3) (end 142.1765 114.3) (width 0.25) (layer B.Cu) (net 13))
 (segment (start 134.5565 111.76) (end 137.0965 111.76) (width 0.25) (layer B.Cu) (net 16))
 (segment (start 140.7795 111.76) (end 141.4145 111.125) (width 0.25) (layer B.Cu) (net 16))
 (segment (start 146.6215 111.125) (end 147.2565 111.76) (width 0.25) (layer B.Cu) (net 16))
 (segment (start 141.4145 111.125) (end 146.6215 111.125) (width 0.25) (layer B.Cu) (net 16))
 (segment (start 137.0965 111.76) (end 140.7795 111.76) (width 0.25) (layer B.Cu) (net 16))
 (segment (start 135.758581 109.22) (end 137.0965 109.22) (width 0.25) (layer B.Cu) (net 19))
 (segment (start 134.5565 109.22) (end 135.758581 109.22) (width 0.25) (layer B.Cu) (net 19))
 (segment (start 137.0965 109.22) (end 142.1765 109.22) (width 0.25) (layer B.Cu) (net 19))
 (segment (start 134.5565 106.68) (end 137.0965 106.68) (width 0.25) (layer B.Cu) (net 22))
 (segment (start 146.80299 106.22649) (end 147.2565 106.68) (width 0.25) (layer B.Cu) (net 22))
 (segment (start 141.5415 105.9815) (end 146.558 105.9815) (width 0.25) (layer B.Cu) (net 22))
 (segment (start 146.558 105.9815) (end 147.2565 106.68) (width 0.25) (layer B.Cu) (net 22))
 (segment (start 137.0965 106.68) (end 140.843 106.68) (width 0.25) (layer B.Cu) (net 22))
 (segment (start 140.843 106.68) (end 141.5415 105.9815) (width 0.25) (layer B.Cu) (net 22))
 (segment (start 134.5565 104.14) (end 137.0965 104.14) (width 0.25) (layer B.Cu) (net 25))
 (segment (start 138.22787 104.14) (end 142.1765 104.14) (width 0.25) (layer B.Cu) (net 25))
 (segment (start 137.0965 104.14) (end 138.22787 104.14) (width 0.25) (layer B.Cu) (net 25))
 (segment (start 152.3365 121.1415) (end 152.3365 121.158) (width 0.25) (layer B.Cu) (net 5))
 (segment (start 151.8465 120.6515) (end 152.3365 121.1415) (width 0.25) (layer B.Cu) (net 5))
 (segment (start 151.8465 119.9515) (end 151.8465 120.6515) (width 0.25) (layer B.Cu) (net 5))
 (segment (start 152.3365 121.92) (end 152.3365 121.158) (width 0.25) (layer B.Cu) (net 5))
 (segment (start 153.39716 121.92) (end 154.8765 121.92) (width 0.25) (layer B.Cu) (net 5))
 (segment (start 152.3365 121.92) (end 153.39716 121.92) (width 0.25) (layer B.Cu) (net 5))
 (segment (start 145.433 117.4115) (end 145.433 117.5565) (width 0.25) (layer B.Cu) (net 8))
 (segment (start 145.433 117.5565) (end 145.923 118.0465) (width 0.25) (layer B.Cu) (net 8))
 (segment (start 145.923 118.0465) (end 147.2565 119.38) (width 0.25) (layer B.Cu) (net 8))
 (segment (start 148.006499 118.630001) (end 147.2565 119.38) (width 0.25) (layer B.Cu) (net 8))
 (segment (start 148.106499 118.530001) (end 148.006499 118.630001) (width 0.25) (layer B.Cu) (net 8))
 (segment (start 154.026501 118.530001) (end 148.106499 118.530001) (width 0.25) (layer B.Cu) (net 8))
 (segment (start 154.8765 119.38) (end 154.026501 118.530001) (width 0.25) (layer B.Cu) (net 8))
 (segment (start 152.3365 115.998) (end 152.3365 116.0145) (width 0.25) (layer B.Cu) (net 11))
 (segment (start 151.8465 115.508) (end 152.3365 115.998) (width 0.25) (layer B.Cu) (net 11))
 (segment (start 151.8465 114.808) (end 151.8465 115.508) (width 0.25) (layer B.Cu) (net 11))
 (segment (start 152.3365 116.7765) (end 152.3365 116.0145) (width 0.25) (layer B.Cu) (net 11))
 (segment (start 152.3365 116.84) (end 154.8765 116.84) (width 0.25) (layer B.Cu) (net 11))
 (segment (start 147.2565 114.3) (end 145.433 112.4765) (width 0.25) (layer B.Cu) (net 14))
 (segment (start 148.106499 113.450001) (end 148.006499 113.550001) (width 0.25) (layer B.Cu) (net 14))
 (segment (start 148.006499 113.550001) (end 147.2565 114.3) (width 0.25) (layer B.Cu) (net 14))
 (segment (start 154.026501 113.450001) (end 148.106499 113.450001) (width 0.25) (layer B.Cu) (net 14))
 (segment (start 154.8765 114.3) (end 154.026501 113.450001) (width 0.25) (layer B.Cu) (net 14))
 (segment (start 152.3365 110.9815) (end 152.3365 110.998) (width 0.25) (layer B.Cu) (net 17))
 (segment (start 151.8465 110.4915) (end 152.3365 110.9815) (width 0.25) (layer B.Cu) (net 17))
 (segment (start 151.8465 109.7915) (end 151.8465 110.4915) (width 0.25) (layer B.Cu) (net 17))
 (segment (start 152.3365 111.76) (end 152.3365 110.998) (width 0.25) (layer B.Cu) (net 17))
 (segment (start 152.3365 111.76) (end 154.8765 111.76) (width 0.25) (layer B.Cu) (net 17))
 (segment (start 145.433 107.3965) (end 145.433 107.2515) (width 0.25) (layer B.Cu) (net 20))
 (segment (start 147.2565 109.22) (end 145.433 107.3965) (width 0.25) (layer B.Cu) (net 20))
 (segment (start 148.006499 108.470001) (end 147.2565 109.22) (width 0.25) (layer B.Cu) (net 20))
 (segment (start 148.106499 108.370001) (end 148.006499 108.470001) (width 0.25) (layer B.Cu) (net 20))
 (segment (start 154.026501 108.370001) (end 148.106499 108.370001) (width 0.25) (layer B.Cu) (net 20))
 (segment (start 154.8765 109.22) (end 154.026501 108.370001) (width 0.25) (layer B.Cu) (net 20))
 (segment (start 152.3365 105.9015) (end 152.3365 105.918) (width 0.25) (layer B.Cu) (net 23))
 (segment (start 151.8465 105.4115) (end 152.3365 105.9015) (width 0.25) (layer B.Cu) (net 23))
 (segment (start 151.8465 104.7115) (end 151.8465 105.4115) (width 0.25) (layer B.Cu) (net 23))
 (segment (start 152.3365 106.68) (end 152.3365 105.918) (width 0.25) (layer B.Cu) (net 23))
 (segment (start 153.39716 106.68) (end 154.8765 106.68) (width 0.25) (layer B.Cu) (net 23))
 (segment (start 152.3365 106.68) (end 153.39716 106.68) (width 0.25) (layer B.Cu) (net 23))
 (segment (start 147.2565 103.3615) (end 147.2565 103.378) (width 0.25) (layer B.Cu) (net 26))
 (segment (start 146.7665 102.8715) (end 147.2565 103.3615) (width 0.25) (layer B.Cu) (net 26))
 (segment (start 146.7665 102.1715) (end 146.7665 102.8715) (width 0.25) (layer B.Cu) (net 26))
 (segment (start 147.2565 104.14) (end 147.2565 103.378) (width 0.25) (layer B.Cu) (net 26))
 (segment (start 153.026501 103.390001) (end 153.7765 104.14) (width 0.25) (layer B.Cu) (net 26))
 (segment (start 153.7765 104.14) (end 154.8765 104.14) (width 0.25) (layer B.Cu) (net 26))
 (segment (start 148.006499 103.390001) (end 153.026501 103.390001) (width 0.25) (layer B.Cu) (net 26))
 (segment (start 147.2565 104.14) (end 148.006499 103.390001) (width 0.25) (layer B.Cu) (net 26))
 (segment (start 147.828 93.98) (end 150.368 93.98) (width 0.25) (layer B.Cu) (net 2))
 (segment (start 144.7165 104.14) (end 144.7165 102.1715) (width 0.25) (layer B.Cu) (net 27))
 (segment (start 140.335 102.1715) (end 139.6365 102.87) (width 0.25) (layer B.Cu) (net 27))
 (segment (start 144.7165 102.1715) (end 140.335 102.1715) (width 0.25) (layer B.Cu) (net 27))
 (segment (start 148.5265 105.41) (end 149.7965 106.68) (width 0.25) (layer B.Cu) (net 24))
 (segment (start 139.6365 105.41) (end 148.5265 105.41) (width 0.25) (layer B.Cu) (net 24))
 (segment (start 149.7965 106.68) (end 149.7965 104.648) (width 0.25) (layer B.Cu) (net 24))
 (segment (start 143.383 107.8865) (end 143.383 107.2515) (width 0.25) (layer B.Cu) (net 21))
 (segment (start 144.7165 109.22) (end 143.383 107.8865) (width 0.25) (layer B.Cu) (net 21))
 (segment (start 139.6365 107.95) (end 140.843 107.95) (width 0.25) (layer B.Cu) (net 21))
 (segment (start 140.843 107.95) (end 141.5415 107.2515) (width 0.25) (layer B.Cu) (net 21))
 (segment (start 143.383 107.2515) (end 141.5415 107.2515) (width 0.25) (layer B.Cu) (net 21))
 (segment (start 139.6365 113.03) (end 140.843 113.03) (width 0.25) (layer B.Cu) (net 15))
 (segment (start 143.383 112.3315) (end 141.5415 112.3315) (width 0.25) (layer B.Cu) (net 15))
 (segment (start 140.843 113.03) (end 141.5415 112.3315) (width 0.25) (layer B.Cu) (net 15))
 (segment (start 149.7965 111.76) (end 149.7965 109.728) (width 0.25) (layer B.Cu) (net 18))
 (segment (start 148.5265 110.49) (end 149.7965 111.76) (width 0.25) (layer B.Cu) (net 18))
 (segment (start 139.6365 110.49) (end 148.5265 110.49) (width 0.25) (layer B.Cu) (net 18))
 (segment (start 143.383 112.9665) (end 143.383 112.3315) (width 0.25) (layer B.Cu) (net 15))
 (segment (start 144.7165 114.3) (end 143.383 112.9665) (width 0.25) (layer B.Cu) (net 15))
 (segment (start 149.7965 114.808) (end 149.7965 116.84) (width 0.25) (layer B.Cu) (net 12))
 (segment (start 139.6365 115.57) (end 149.0345 115.57) (width 0.25) (layer B.Cu) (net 12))
 (segment (start 149.0345 115.57) (end 149.7965 114.808) (width 0.25) (layer B.Cu) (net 12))
 (segment (start 143.383 117.4115) (end 143.383 117.5385) (width 0.25) (layer B.Cu) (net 9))
 (segment (start 144.7165 118.872) (end 144.7165 119.38) (width 0.25) (layer B.Cu) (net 9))
 (segment (start 143.383 117.5385) (end 144.7165 118.872) (width 0.25) (layer B.Cu) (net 9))
 (segment (start 142.5575 117.4115) (end 143.383 117.4115) (width 0.25) (layer B.Cu) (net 9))
 (segment (start 141.9225 117.4115) (end 142.5575 117.4115) (width 0.25) (layer B.Cu) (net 9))
 (segment (start 139.6365 118.11) (end 141.224 118.11) (width 0.25) (layer B.Cu) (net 9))
 (segment (start 141.224 118.11) (end 141.9225 117.4115) (width 0.25) (layer B.Cu) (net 9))
 (segment (start 148.844 119.9515) (end 149.7965 119.9515) (width 0.25) (layer B.Cu) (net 6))
 (segment (start 149.7965 121.92) (end 149.7965 119.9515) (width 0.25) (layer B.Cu) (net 6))
 (segment (start 148.1455 120.65) (end 148.844 119.9515) (width 0.25) (layer B.Cu) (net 6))
 (segment (start 139.6365 120.65) (end 148.1455 120.65) (width 0.25) (layer B.Cu) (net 6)))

